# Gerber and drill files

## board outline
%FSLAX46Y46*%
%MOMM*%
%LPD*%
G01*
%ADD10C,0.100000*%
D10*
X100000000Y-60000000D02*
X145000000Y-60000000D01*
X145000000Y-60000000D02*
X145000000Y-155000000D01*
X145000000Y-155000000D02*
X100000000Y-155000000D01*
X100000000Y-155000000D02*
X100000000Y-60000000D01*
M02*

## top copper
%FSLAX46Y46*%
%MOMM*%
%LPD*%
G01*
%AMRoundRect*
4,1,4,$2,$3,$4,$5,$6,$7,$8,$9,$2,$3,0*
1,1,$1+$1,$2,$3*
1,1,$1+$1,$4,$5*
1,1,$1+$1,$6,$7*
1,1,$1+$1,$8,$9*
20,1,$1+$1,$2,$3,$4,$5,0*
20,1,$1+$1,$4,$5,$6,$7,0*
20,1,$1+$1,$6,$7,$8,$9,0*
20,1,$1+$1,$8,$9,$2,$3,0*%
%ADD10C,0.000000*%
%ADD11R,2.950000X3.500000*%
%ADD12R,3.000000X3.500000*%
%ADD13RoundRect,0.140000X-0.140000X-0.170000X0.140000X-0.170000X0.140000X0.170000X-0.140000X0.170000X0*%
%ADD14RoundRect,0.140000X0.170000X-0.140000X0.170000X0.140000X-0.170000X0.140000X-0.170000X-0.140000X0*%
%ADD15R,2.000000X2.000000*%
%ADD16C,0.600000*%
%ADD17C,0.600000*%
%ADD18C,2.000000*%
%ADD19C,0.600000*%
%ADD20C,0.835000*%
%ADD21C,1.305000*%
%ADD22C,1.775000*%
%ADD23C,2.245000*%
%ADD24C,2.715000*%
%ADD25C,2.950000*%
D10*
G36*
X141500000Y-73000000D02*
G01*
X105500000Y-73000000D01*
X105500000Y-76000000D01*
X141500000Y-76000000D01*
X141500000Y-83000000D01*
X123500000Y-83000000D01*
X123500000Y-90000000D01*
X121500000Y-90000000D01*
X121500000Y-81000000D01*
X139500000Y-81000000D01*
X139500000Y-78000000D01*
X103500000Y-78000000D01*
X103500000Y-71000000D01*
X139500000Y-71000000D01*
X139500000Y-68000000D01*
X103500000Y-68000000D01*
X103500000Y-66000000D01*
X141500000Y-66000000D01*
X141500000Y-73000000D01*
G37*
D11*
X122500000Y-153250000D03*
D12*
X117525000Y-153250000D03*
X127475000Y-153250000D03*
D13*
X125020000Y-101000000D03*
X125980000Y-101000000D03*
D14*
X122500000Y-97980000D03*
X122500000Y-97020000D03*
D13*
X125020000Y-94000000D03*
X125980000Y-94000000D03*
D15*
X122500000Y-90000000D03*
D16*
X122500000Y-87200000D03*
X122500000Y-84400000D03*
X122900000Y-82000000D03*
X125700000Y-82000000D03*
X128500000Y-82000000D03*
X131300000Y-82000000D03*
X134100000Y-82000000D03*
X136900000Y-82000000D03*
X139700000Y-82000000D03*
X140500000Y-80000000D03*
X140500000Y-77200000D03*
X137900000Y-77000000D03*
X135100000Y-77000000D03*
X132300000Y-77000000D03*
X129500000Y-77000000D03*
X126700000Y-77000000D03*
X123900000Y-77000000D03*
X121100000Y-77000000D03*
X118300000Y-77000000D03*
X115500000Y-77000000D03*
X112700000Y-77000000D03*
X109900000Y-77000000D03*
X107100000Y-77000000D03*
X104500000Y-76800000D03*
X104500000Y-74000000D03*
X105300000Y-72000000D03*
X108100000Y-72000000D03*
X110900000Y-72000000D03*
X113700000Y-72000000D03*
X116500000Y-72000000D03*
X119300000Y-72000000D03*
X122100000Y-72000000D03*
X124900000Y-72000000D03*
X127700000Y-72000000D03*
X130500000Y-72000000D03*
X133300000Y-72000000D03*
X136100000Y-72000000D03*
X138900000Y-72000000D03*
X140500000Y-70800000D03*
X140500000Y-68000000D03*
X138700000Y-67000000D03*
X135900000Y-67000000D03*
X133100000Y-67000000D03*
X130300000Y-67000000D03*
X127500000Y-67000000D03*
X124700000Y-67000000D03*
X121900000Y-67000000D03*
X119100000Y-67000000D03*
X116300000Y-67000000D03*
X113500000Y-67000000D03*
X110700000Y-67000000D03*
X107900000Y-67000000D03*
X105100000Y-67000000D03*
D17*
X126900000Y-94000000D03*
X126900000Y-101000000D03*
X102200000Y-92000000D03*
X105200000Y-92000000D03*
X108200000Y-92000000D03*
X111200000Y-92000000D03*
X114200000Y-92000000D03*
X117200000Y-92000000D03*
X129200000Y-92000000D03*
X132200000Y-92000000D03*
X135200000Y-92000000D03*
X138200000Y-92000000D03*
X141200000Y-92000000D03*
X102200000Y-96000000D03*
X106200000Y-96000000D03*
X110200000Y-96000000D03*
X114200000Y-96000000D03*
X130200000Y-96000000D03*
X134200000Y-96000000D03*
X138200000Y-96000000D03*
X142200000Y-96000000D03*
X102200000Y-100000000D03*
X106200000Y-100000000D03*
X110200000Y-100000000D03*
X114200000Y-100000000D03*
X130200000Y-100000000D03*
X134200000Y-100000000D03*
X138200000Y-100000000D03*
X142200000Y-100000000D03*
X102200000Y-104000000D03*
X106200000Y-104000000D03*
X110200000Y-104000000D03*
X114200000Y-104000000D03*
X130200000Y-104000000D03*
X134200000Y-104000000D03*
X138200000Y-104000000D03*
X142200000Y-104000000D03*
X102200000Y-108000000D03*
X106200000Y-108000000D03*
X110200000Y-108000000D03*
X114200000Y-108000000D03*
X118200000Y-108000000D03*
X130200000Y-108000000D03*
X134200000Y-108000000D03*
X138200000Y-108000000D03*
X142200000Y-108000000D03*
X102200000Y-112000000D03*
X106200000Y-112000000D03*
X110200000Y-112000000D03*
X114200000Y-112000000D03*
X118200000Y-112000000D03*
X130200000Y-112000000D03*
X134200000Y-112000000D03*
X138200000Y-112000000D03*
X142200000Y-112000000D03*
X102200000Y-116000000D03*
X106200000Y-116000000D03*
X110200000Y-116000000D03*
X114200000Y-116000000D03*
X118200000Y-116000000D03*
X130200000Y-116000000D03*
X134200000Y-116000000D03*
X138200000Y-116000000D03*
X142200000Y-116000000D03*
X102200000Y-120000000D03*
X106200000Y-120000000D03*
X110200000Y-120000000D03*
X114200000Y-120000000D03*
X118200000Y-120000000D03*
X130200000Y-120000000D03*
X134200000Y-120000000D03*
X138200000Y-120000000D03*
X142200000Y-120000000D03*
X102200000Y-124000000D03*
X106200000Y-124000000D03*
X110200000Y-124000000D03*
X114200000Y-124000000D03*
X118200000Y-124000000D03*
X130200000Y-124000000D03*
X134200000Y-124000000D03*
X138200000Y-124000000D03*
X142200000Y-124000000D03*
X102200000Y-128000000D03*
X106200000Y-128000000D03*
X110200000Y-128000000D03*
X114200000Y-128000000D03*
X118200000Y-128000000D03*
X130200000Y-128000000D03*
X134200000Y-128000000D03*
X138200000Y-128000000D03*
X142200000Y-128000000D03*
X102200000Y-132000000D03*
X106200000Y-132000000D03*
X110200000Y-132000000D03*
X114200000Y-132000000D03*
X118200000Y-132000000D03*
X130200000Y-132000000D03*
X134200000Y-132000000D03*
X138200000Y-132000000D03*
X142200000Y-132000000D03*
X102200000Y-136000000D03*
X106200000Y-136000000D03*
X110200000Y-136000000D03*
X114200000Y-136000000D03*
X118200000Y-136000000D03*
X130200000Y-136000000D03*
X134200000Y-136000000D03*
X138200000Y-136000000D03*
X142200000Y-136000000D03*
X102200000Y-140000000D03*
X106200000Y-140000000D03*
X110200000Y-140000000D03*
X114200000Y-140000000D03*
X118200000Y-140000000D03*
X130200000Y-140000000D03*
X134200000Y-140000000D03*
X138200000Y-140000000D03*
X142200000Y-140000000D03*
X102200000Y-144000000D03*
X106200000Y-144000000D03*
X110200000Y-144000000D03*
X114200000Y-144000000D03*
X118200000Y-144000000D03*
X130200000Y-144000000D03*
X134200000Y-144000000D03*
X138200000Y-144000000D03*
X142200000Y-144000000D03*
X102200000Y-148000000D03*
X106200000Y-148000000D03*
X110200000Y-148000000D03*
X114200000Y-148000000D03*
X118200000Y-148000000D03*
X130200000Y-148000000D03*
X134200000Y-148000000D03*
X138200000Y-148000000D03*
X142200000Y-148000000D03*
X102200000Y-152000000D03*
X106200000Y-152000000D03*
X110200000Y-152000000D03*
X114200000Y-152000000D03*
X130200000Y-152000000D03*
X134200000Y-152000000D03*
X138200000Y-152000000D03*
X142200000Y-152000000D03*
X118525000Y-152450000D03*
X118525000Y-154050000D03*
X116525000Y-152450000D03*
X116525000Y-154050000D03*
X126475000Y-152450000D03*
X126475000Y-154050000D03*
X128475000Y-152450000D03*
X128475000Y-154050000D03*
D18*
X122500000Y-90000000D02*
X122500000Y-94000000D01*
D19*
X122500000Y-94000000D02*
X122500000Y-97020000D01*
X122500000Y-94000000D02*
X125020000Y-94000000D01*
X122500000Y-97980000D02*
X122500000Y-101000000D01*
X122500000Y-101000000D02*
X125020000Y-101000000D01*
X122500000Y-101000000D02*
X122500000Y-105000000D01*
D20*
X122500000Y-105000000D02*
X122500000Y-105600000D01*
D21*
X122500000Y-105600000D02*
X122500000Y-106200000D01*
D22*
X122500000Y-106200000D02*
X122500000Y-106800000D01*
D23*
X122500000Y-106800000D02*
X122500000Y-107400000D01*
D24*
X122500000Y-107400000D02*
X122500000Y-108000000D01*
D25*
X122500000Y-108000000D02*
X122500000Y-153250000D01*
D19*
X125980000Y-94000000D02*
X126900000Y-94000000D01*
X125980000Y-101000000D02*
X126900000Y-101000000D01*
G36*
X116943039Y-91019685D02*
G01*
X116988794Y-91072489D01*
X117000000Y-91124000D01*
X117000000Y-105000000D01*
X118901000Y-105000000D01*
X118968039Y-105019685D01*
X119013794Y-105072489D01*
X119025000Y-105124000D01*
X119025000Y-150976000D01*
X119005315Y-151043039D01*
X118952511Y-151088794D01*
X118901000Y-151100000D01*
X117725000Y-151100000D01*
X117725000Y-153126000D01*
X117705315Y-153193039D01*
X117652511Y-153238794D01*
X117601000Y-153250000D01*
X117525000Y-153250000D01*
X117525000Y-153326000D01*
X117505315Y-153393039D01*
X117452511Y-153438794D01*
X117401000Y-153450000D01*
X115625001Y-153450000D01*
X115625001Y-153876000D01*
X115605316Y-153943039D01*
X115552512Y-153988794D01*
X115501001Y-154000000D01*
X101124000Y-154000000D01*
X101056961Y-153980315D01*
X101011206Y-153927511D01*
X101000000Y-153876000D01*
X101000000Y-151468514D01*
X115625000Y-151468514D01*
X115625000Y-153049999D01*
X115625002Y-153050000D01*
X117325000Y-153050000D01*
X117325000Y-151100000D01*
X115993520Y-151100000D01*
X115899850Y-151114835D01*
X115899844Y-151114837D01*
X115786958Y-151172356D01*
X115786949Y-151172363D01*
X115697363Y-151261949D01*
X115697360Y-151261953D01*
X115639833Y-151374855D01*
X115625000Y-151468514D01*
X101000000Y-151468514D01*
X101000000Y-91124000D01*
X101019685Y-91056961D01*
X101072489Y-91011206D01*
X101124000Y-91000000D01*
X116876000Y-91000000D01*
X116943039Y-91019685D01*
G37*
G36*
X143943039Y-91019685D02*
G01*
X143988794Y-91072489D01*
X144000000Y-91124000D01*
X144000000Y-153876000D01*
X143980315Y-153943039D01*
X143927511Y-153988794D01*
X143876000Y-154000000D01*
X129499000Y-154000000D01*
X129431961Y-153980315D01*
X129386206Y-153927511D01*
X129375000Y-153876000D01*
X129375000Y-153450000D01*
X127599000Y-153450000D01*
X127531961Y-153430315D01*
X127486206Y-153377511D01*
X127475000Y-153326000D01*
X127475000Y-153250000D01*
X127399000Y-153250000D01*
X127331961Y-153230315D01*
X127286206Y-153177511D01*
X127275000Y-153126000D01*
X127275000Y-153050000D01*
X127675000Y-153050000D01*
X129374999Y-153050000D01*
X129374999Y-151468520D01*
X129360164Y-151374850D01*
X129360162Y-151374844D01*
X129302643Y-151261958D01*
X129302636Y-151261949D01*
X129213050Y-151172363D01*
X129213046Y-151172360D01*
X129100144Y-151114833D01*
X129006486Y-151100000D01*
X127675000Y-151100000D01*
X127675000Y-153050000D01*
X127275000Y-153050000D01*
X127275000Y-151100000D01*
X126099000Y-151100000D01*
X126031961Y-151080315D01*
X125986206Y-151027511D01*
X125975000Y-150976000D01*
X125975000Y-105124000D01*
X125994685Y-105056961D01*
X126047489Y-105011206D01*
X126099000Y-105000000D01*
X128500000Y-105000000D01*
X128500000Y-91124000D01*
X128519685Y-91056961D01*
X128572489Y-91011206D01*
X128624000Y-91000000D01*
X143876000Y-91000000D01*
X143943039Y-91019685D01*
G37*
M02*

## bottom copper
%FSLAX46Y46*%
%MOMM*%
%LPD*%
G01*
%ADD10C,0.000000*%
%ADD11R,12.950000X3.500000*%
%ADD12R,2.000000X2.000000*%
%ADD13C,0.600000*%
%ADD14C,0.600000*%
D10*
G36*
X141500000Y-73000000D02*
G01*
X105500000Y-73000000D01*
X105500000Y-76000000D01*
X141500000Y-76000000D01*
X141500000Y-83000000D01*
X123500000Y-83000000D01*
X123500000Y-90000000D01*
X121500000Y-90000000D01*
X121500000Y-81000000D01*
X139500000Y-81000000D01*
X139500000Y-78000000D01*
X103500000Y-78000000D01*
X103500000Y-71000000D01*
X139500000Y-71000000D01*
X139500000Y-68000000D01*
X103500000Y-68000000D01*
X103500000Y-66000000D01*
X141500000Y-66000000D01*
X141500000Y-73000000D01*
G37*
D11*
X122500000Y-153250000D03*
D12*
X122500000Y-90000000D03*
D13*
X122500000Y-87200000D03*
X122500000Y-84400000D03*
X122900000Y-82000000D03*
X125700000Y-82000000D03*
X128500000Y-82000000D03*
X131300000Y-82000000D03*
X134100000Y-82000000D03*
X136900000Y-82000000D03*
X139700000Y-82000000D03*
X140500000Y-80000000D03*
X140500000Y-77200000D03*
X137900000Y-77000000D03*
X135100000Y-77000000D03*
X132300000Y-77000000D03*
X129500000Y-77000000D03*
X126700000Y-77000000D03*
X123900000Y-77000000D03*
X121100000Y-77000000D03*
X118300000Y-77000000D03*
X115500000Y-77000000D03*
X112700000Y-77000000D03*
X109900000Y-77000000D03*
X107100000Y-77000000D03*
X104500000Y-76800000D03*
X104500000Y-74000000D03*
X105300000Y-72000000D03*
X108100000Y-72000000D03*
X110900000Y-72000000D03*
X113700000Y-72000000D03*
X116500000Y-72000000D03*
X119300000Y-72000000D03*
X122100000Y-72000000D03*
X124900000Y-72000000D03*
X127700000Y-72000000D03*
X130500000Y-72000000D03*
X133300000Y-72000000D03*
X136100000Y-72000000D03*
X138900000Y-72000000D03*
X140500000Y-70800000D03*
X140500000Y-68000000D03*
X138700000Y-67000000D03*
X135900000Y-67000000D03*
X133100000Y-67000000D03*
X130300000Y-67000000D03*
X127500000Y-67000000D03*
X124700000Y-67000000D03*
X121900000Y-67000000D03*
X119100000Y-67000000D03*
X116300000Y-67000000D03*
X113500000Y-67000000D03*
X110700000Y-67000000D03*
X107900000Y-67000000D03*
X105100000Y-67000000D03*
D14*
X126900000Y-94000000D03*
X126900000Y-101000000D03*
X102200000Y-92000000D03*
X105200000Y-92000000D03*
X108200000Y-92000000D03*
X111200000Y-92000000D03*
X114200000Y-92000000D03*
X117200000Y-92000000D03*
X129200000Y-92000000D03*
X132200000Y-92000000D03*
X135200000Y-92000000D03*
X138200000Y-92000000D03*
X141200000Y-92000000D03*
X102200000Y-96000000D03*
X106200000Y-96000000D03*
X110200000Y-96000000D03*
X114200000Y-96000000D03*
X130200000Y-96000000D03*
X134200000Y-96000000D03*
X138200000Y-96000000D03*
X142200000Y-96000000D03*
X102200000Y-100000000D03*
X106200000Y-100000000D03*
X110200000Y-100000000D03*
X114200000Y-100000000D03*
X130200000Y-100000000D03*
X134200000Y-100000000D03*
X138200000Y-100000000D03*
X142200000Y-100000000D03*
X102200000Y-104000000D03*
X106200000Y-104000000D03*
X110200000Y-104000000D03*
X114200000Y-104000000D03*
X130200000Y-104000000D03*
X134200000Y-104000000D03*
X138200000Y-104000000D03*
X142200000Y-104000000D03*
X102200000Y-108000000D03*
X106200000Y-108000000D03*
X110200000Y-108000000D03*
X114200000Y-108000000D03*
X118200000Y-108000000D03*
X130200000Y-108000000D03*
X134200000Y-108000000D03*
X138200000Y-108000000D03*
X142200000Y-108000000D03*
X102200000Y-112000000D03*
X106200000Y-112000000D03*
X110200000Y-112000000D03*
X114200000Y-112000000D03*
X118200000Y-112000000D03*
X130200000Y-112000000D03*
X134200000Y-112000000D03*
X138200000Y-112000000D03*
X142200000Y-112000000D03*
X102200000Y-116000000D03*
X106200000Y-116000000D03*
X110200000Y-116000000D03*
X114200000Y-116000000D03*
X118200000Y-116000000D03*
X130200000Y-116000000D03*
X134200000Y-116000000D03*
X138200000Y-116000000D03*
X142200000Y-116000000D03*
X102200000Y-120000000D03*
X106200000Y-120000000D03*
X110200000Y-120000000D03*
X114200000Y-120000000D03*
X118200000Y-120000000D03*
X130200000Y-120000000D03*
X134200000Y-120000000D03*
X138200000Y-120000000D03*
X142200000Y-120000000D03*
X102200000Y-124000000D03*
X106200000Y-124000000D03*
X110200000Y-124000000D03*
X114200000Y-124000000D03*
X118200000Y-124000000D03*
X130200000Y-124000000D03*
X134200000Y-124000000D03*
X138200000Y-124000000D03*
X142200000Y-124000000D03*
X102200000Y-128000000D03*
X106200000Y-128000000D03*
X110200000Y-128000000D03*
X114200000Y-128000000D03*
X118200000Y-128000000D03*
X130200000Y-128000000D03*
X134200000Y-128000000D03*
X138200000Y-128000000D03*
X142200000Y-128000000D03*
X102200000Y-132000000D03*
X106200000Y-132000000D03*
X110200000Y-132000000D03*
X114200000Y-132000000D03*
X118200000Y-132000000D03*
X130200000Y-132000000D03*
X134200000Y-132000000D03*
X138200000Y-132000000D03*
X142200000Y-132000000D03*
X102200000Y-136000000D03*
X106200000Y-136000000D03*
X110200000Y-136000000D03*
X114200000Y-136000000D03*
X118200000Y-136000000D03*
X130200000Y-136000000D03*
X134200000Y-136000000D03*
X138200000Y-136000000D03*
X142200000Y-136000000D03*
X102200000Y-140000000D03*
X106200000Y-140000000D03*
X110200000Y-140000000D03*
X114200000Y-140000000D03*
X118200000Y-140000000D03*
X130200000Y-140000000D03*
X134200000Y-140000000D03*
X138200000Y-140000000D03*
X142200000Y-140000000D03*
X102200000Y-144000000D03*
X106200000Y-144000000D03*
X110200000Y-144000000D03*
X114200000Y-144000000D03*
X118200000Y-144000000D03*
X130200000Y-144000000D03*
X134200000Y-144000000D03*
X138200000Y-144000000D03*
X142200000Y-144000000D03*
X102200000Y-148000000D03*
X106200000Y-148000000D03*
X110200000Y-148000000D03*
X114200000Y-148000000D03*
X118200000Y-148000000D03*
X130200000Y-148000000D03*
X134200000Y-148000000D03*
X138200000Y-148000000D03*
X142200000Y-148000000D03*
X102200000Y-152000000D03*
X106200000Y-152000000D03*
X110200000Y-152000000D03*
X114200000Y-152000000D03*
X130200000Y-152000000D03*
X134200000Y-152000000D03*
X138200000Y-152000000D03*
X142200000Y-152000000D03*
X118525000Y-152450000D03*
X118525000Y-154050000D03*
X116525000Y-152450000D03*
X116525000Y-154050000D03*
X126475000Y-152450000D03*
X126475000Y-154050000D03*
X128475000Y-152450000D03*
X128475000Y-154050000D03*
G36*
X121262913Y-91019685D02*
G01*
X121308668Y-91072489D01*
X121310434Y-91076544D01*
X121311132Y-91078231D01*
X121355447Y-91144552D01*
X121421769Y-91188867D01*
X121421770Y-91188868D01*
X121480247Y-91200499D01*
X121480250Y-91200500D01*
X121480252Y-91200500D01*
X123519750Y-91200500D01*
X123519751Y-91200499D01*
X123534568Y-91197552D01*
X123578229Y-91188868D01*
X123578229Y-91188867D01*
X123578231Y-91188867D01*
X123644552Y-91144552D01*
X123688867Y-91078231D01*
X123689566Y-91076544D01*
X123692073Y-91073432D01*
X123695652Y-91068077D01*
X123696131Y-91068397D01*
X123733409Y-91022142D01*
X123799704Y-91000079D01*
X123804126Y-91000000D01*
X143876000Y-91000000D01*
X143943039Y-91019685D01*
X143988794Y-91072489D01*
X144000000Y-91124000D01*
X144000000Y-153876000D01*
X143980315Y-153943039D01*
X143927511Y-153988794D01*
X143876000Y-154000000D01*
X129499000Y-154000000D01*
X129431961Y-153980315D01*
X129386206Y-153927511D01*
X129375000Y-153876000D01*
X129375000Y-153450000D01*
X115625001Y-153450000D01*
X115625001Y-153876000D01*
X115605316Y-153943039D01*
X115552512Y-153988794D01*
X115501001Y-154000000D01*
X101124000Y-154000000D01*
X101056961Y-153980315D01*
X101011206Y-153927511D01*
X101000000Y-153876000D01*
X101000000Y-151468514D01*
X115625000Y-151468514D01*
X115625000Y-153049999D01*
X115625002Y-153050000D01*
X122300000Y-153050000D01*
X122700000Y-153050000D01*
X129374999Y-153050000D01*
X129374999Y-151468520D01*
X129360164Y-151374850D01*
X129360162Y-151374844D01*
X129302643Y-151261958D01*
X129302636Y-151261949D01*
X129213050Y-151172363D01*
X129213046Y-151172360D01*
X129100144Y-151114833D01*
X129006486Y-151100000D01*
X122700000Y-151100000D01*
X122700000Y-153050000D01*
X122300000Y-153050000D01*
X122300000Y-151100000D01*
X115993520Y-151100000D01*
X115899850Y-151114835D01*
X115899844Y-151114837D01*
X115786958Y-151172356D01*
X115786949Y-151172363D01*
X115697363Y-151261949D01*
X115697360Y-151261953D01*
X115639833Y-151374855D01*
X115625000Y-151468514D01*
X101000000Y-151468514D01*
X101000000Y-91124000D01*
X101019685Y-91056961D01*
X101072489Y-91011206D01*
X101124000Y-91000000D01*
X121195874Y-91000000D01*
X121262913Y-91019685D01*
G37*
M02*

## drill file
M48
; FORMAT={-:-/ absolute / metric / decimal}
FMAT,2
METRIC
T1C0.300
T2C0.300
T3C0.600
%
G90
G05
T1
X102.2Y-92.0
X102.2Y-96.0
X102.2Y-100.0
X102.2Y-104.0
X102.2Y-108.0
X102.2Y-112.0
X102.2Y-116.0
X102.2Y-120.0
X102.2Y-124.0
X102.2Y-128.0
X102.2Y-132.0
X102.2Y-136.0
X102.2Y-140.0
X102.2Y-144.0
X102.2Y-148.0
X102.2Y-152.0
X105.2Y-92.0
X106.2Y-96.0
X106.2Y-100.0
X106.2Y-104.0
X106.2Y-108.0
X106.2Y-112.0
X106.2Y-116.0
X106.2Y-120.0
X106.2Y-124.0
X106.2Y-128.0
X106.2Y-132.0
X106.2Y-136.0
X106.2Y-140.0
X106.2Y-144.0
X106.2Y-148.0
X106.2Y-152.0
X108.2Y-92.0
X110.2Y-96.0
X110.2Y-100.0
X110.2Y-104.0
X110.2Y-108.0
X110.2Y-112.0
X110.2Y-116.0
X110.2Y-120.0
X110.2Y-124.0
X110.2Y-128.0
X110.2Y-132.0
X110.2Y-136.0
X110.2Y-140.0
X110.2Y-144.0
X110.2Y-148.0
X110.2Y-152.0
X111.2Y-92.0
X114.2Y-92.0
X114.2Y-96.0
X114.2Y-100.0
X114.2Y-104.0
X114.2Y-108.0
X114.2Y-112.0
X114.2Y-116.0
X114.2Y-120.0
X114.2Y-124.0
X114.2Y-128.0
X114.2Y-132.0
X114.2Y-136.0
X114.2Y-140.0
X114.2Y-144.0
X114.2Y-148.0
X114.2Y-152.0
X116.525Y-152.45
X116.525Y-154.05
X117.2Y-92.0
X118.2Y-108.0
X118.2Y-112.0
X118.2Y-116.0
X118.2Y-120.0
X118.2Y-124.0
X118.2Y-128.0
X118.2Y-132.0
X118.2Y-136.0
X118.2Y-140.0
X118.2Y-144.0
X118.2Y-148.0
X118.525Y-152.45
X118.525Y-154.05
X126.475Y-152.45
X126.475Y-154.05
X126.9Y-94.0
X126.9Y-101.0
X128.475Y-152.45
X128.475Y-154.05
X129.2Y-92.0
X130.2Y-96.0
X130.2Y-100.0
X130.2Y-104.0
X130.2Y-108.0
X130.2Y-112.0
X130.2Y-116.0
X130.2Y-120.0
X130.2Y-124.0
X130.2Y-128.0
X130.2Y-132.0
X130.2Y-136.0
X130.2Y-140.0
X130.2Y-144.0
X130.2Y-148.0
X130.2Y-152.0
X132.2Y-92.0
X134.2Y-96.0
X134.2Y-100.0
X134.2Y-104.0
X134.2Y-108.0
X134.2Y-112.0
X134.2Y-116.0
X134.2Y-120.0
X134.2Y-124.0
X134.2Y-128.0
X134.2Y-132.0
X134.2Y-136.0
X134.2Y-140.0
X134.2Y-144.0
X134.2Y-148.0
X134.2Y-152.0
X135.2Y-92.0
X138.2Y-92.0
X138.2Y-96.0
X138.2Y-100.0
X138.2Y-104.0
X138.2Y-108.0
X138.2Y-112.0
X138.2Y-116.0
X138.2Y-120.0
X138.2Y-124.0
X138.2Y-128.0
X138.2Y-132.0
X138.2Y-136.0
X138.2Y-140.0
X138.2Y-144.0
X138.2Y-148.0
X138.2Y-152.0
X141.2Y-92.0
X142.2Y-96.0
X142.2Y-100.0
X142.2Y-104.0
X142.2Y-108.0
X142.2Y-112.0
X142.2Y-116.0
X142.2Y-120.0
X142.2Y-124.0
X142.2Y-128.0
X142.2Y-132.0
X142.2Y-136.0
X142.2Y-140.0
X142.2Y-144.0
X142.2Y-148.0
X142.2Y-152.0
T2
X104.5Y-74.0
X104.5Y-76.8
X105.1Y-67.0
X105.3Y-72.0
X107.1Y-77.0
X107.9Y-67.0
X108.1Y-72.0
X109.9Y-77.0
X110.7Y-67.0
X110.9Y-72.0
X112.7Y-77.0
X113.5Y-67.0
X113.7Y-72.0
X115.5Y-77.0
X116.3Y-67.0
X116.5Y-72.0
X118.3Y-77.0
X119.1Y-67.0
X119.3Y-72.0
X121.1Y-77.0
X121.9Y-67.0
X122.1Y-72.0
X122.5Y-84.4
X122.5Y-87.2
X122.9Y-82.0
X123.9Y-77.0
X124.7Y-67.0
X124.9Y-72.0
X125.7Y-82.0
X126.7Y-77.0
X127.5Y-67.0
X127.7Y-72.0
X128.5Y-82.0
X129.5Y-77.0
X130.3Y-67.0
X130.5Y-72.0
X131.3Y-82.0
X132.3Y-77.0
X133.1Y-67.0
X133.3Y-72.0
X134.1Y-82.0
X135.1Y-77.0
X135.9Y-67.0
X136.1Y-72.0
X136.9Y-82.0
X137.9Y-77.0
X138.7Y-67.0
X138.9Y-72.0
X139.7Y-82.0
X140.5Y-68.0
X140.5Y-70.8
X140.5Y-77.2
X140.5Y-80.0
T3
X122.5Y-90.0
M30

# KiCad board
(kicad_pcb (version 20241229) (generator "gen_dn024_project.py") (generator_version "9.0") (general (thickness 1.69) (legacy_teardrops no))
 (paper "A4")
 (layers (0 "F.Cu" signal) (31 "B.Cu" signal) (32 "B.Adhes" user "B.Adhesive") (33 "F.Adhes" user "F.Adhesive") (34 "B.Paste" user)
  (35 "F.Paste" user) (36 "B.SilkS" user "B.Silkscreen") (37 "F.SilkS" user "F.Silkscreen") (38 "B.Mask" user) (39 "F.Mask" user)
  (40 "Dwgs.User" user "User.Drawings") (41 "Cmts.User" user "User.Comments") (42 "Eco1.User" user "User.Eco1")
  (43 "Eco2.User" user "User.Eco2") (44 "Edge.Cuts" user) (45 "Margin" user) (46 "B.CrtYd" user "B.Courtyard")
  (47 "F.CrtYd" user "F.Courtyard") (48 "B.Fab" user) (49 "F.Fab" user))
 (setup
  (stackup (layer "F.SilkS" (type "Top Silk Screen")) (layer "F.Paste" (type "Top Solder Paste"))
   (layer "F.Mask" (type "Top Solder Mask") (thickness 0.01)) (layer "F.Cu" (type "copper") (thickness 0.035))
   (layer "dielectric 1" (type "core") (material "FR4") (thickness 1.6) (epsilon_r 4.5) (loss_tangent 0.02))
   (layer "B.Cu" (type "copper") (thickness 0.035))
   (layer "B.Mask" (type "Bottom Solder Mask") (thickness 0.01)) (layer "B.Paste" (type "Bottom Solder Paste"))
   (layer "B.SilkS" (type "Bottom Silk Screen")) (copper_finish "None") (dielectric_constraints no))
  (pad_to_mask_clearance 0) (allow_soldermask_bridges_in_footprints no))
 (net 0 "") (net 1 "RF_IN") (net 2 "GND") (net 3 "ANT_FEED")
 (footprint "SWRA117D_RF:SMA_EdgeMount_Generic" (layer "F.Cu") (at 122.5 155 90)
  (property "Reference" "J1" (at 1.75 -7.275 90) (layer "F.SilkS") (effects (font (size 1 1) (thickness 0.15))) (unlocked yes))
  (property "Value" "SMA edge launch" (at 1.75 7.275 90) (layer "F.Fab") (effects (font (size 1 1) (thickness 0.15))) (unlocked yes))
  (pad "1" smd rect (at 1.75 0 90) (size 3.5 2.95) (layers "F.Cu" "F.Paste" "F.Mask") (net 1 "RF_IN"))
  (pad "2" smd rect (at 1.75 -4.975 90) (size 3.5 3) (layers "F.Cu" "F.Paste" "F.Mask") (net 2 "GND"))
  (pad "2" smd rect (at 1.75 4.975 90) (size 3.5 3) (layers "F.Cu" "F.Paste" "F.Mask") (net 2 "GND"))
  (pad "2" smd rect (at 1.75 0 90) (size 3.5 12.95) (layers "B.Cu" "B.Paste" "B.Mask") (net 2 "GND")))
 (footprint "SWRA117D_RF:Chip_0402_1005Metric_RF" (layer "F.Cu") (at 125.5 101)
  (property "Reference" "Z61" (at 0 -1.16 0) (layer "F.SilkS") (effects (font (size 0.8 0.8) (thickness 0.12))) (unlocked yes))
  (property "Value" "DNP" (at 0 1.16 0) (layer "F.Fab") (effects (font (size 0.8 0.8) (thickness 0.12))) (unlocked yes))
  (pad "1" smd roundrect (at -0.48 0) (size 0.56 0.62) (layers "F.Cu" "F.Paste" "F.Mask") (roundrect_rratio 0.25) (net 1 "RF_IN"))
  (pad "2" smd roundrect (at 0.48 0) (size 0.56 0.62) (layers "F.Cu" "F.Paste" "F.Mask") (roundrect_rratio 0.25) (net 2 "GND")))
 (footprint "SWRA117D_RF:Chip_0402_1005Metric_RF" (layer "F.Cu") (at 122.5 97.5 90)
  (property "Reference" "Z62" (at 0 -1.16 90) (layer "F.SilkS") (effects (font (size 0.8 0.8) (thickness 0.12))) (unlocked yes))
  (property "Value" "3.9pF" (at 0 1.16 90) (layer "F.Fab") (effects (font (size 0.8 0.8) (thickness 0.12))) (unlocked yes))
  (pad "1" smd roundrect (at -0.48 0 90) (size 0.56 0.62) (layers "F.Cu" "F.Paste" "F.Mask") (roundrect_rratio 0.25) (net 1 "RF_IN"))
  (pad "2" smd roundrect (at 0.48 0 90) (size 0.56 0.62) (layers "F.Cu" "F.Paste" "F.Mask") (roundrect_rratio 0.25) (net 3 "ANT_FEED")))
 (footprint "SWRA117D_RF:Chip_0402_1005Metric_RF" (layer "F.Cu") (at 125.5 94)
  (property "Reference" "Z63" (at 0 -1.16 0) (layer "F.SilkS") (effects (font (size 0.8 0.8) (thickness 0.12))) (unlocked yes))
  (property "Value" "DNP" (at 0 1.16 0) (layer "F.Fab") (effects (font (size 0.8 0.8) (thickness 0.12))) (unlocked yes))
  (pad "1" smd roundrect (at -0.48 0) (size 0.56 0.62) (layers "F.Cu" "F.Paste" "F.Mask") (roundrect_rratio 0.25) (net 3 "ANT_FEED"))
  (pad "2" smd roundrect (at 0.48 0) (size 0.56 0.62) (layers "F.Cu" "F.Paste" "F.Mask") (roundrect_rratio 0.25) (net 2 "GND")))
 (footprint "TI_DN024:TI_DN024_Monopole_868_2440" (layer "F.Cu") (at 122.5 90)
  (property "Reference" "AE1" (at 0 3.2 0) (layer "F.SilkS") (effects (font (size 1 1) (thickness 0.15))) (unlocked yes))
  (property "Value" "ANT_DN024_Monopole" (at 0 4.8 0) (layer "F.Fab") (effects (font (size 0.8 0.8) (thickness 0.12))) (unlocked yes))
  (fp_poly
   (pts (xy 1 0) (xy 1 -7) (xy 19 -7) (xy 19 -14) (xy -17 -14) (xy -17 -17) (xy 19 -17) (xy 19 -24) (xy -19 -24) (xy -19 -22) (xy 17 -22)
    (xy 17 -19) (xy -19 -19) (xy -19 -12) (xy 17 -12) (xy 17 -9) (xy -1 -9) (xy -1 0))
   (stroke (width 0) (type solid)) (fill yes) (layer "F.Cu"))
  (fp_poly
   (pts (xy 1 0) (xy 1 -7) (xy 19 -7) (xy 19 -14) (xy -17 -14) (xy -17 -17) (xy 19 -17) (xy 19 -24) (xy -19 -24) (xy -19 -22) (xy 17 -22)
    (xy 17 -19) (xy -19 -19) (xy -19 -12) (xy 17 -12) (xy 17 -9) (xy -1 -9) (xy -1 0))
   (stroke (width 0) (type solid)) (fill yes) (layer "B.Cu"))
  (pad "1" thru_hole rect (at 0 0) (size 2 2) (drill 0.6) (layers "*.Cu" "*.Mask") (remove_unused_layers no) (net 3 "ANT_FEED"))
  (pad "1" thru_hole circle (at 0 -2.8) (size 0.6 0.6) (drill 0.3) (layers "*.Cu") (remove_unused_layers no) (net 3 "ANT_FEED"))
  (pad "1" thru_hole circle (at 0 -5.6) (size 0.6 0.6) (drill 0.3) (layers "*.Cu") (remove_unused_layers no) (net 3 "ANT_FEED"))
  (pad "1" thru_hole circle (at 0.4 -8) (size 0.6 0.6) (drill 0.3) (layers "*.Cu") (remove_unused_layers no) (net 3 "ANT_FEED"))
  (pad "1" thru_hole circle (at 3.2 -8) (size 0.6 0.6) (drill 0.3) (layers "*.Cu") (remove_unused_layers no) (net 3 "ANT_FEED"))
  (pad "1" thru_hole circle (at 6 -8) (size 0.6 0.6) (drill 0.3) (layers "*.Cu") (remove_unused_layers no) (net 3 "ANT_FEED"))
  (pad "1" thru_hole circle (at 8.8 -8) (size 0.6 0.6) (drill 0.3) (layers "*.Cu") (remove_unused_layers no) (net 3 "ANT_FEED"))
  (pad "1" thru_hole circle (at 11.6 -8) (size 0.6 0.6) (drill 0.3) (layers "*.Cu") (remove_unused_layers no) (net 3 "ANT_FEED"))
  (pad "1" thru_hole circle (at 14.4 -8) (size 0.6 0.6) (drill 0.3) (layers "*.Cu") (remove_unused_layers no) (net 3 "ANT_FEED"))
  (pad "1" thru_hole circle (at 17.2 -8) (size 0.6 0.6) (drill 0.3) (layers "*.Cu") (remove_unused_layers no) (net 3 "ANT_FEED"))
  (pad "1" thru_hole circle (at 18 -10) (size 0.6 0.6) (drill 0.3) (layers "*.Cu") (remove_unused_layers no) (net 3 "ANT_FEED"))
  (pad "1" thru_hole circle (at 18 -12.8) (size 0.6 0.6) (drill 0.3) (layers "*.Cu") (remove_unused_layers no) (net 3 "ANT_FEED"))
  (pad "1" thru_hole circle (at 15.4 -13) (size 0.6 0.6) (drill 0.3) (layers "*.Cu") (remove_unused_layers no) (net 3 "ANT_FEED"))
  (pad "1" thru_hole circle (at 12.6 -13) (size 0.6 0.6) (drill 0.3) (layers "*.Cu") (remove_unused_layers no) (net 3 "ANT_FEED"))
  (pad "1" thru_hole circle (at 9.8 -13) (size 0.6 0.6) (drill 0.3) (layers "*.Cu") (remove_unused_layers no) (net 3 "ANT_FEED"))
  (pad "1" thru_hole circle (at 7 -13) (size 0.6 0.6) (drill 0.3) (layers "*.Cu") (remove_unused_layers no) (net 3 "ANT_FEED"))
  (pad "1" thru_hole circle (at 4.2 -13) (size 0.6 0.6) (drill 0.3) (layers "*.Cu") (remove_unused_layers no) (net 3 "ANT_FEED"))
  (pad "1" thru_hole circle (at 1.4 -13) (size 0.6 0.6) (drill 0.3) (layers "*.Cu") (remove_unused_layers no) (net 3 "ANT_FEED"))
  (pad "1" thru_hole circle (at -1.4 -13) (size 0.6 0.6) (drill 0.3) (layers "*.Cu") (remove_unused_layers no) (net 3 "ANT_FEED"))
  (pad "1" thru_hole circle (at -4.2 -13) (size 0.6 0.6) (drill 0.3) (layers "*.Cu") (remove_unused_layers no) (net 3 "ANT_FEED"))
  (pad "1" thru_hole circle (at -7 -13) (size 0.6 0.6) (drill 0.3) (layers "*.Cu") (remove_unused_layers no) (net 3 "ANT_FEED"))
  (pad "1" thru_hole circle (at -9.8 -13) (size 0.6 0.6) (drill 0.3) (layers "*.Cu") (remove_unused_layers no) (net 3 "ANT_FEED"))
  (pad "1" thru_hole circle (at -12.6 -13) (size 0.6 0.6) (drill 0.3) (layers "*.Cu") (remove_unused_layers no) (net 3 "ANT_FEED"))
  (pad "1" thru_hole circle (at -15.4 -13) (size 0.6 0.6) (drill 0.3) (layers "*.Cu") (remove_unused_layers no) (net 3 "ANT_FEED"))
  (pad "1" thru_hole circle (at -18 -13.2) (size 0.6 0.6) (drill 0.3) (layers "*.Cu") (remove_unused_layers no) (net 3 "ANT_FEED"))
  (pad "1" thru_hole circle (at -18 -16) (size 0.6 0.6) (drill 0.3) (layers "*.Cu") (remove_unused_layers no) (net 3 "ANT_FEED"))
  (pad "1" thru_hole circle (at -17.2 -18) (size 0.6 0.6) (drill 0.3) (layers "*.Cu") (remove_unused_layers no) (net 3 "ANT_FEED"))
  (pad "1" thru_hole circle (at -14.4 -18) (size 0.6 0.6) (drill 0.3) (layers "*.Cu") (remove_unused_layers no) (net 3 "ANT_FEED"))
  (pad "1" thru_hole circle (at -11.6 -18) (size 0.6 0.6) (drill 0.3) (layers "*.Cu") (remove_unused_layers no) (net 3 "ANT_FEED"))
  (pad "1" thru_hole circle (at -8.8 -18) (size 0.6 0.6) (drill 0.3) (layers "*.Cu") (remove_unused_layers no) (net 3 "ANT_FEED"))
  (pad "1" thru_hole circle (at -6 -18) (size 0.6 0.6) (drill 0.3) (layers "*.Cu") (remove_unused_layers no) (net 3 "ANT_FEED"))
  (pad "1" thru_hole circle (at -3.2 -18) (size 0.6 0.6) (drill 0.3) (layers "*.Cu") (remove_unused_layers no) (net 3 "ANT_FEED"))
  (pad "1" thru_hole circle (at -0.4 -18) (size 0.6 0.6) (drill 0.3) (layers "*.Cu") (remove_unused_layers no) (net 3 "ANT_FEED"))
  (pad "1" thru_hole circle (at 2.4 -18) (size 0.6 0.6) (drill 0.3) (layers "*.Cu") (remove_unused_layers no) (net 3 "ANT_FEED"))
  (pad "1" thru_hole circle (at 5.2 -18) (size 0.6 0.6) (drill 0.3) (layers "*.Cu") (remove_unused_layers no) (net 3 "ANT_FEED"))
  (pad "1" thru_hole circle (at 8 -18) (size 0.6 0.6) (drill 0.3) (layers "*.Cu") (remove_unused_layers no) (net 3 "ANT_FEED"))
  (pad "1" thru_hole circle (at 10.8 -18) (size 0.6 0.6) (drill 0.3) (layers "*.Cu") (remove_unused_layers no) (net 3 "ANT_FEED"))
  (pad "1" thru_hole circle (at 13.6 -18) (size 0.6 0.6) (drill 0.3) (layers "*.Cu") (remove_unused_layers no) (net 3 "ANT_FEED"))
  (pad "1" thru_hole circle (at 16.4 -18) (size 0.6 0.6) (drill 0.3) (layers "*.Cu") (remove_unused_layers no) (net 3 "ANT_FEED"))
  (pad "1" thru_hole circle (at 18 -19.2) (size 0.6 0.6) (drill 0.3) (layers "*.Cu") (remove_unused_layers no) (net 3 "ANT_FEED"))
  (pad "1" thru_hole circle (at 18 -22) (size 0.6 0.6) (drill 0.3) (layers "*.Cu") (remove_unused_layers no) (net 3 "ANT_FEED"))
  (pad "1" thru_hole circle (at 16.2 -23) (size 0.6 0.6) (drill 0.3) (layers "*.Cu") (remove_unused_layers no) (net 3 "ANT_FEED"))
  (pad "1" thru_hole circle (at 13.4 -23) (size 0.6 0.6) (drill 0.3) (layers "*.Cu") (remove_unused_layers no) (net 3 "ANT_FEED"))
  (pad "1" thru_hole circle (at 10.6 -23) (size 0.6 0.6) (drill 0.3) (layers "*.Cu") (remove_unused_layers no) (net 3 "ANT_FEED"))
  (pad "1" thru_hole circle (at 7.8 -23) (size 0.6 0.6) (drill 0.3) (layers "*.Cu") (remove_unused_layers no) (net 3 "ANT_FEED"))
  (pad "1" thru_hole circle (at 5 -23) (size 0.6 0.6) (drill 0.3) (layers "*.Cu") (remove_unused_layers no) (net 3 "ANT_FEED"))
  (pad "1" thru_hole circle (at 2.2 -23) (size 0.6 0.6) (drill 0.3) (layers "*.Cu") (remove_unused_layers no) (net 3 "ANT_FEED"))
  (pad "1" thru_hole circle (at -0.6 -23) (size 0.6 0.6) (drill 0.3) (layers "*.Cu") (remove_unused_layers no) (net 3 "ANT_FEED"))
  (pad "1" thru_hole circle (at -3.4 -23) (size 0.6 0.6) (drill 0.3) (layers "*.Cu") (remove_unused_layers no) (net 3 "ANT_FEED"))
  (pad "1" thru_hole circle (at -6.2 -23) (size 0.6 0.6) (drill 0.3) (layers "*.Cu") (remove_unused_layers no) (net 3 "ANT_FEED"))
  (pad "1" thru_hole circle (at -9 -23) (size 0.6 0.6) (drill 0.3) (layers "*.Cu") (remove_unused_layers no) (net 3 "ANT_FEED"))
  (pad "1" thru_hole circle (at -11.8 -23) (size 0.6 0.6) (drill 0.3) (layers "*.Cu") (remove_unused_layers no) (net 3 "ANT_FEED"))
  (pad "1" thru_hole circle (at -14.6 -23) (size 0.6 0.6) (drill 0.3) (layers "*.Cu") (remove_unused_layers no) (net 3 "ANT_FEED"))
  (pad "1" thru_hole circle (at -17.4 -23) (size 0.6 0.6) (drill 0.3) (layers "*.Cu") (remove_unused_layers no) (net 3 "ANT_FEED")))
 (gr_line (start 100 60) (end 145 60) (stroke (width 0.1) (type solid)) (layer "Edge.Cuts"))
 (gr_line (start 145 60) (end 145 155) (stroke (width 0.1) (type solid)) (layer "Edge.Cuts"))
 (gr_line (start 145 155) (end 100 155) (stroke (width 0.1) (type solid)) (layer "Edge.Cuts"))
 (gr_line (start 100 155) (end 100 60) (stroke (width 0.1) (type solid)) (layer "Edge.Cuts"))
 (segment (start 122.5 90) (end 122.5 94) (width 2) (layer "F.Cu") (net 3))
 (segment (start 122.5 94) (end 122.5 97.02) (width 0.6) (layer "F.Cu") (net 3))
 (segment (start 122.5 94) (end 125.02 94) (width 0.6) (layer "F.Cu") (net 3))
 (segment (start 122.5 97.98) (end 122.5 101) (width 0.6) (layer "F.Cu") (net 1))
 (segment (start 122.5 101) (end 125.02 101) (width 0.6) (layer "F.Cu") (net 1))
 (segment (start 122.5 101) (end 122.5 105) (width 0.6) (layer "F.Cu") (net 1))
 (segment (start 122.5 105) (end 122.5 105.6) (width 0.835) (layer "F.Cu") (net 1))
 (segment (start 122.5 105.6) (end 122.5 106.2) (width 1.305) (layer "F.Cu") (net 1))
 (segment (start 122.5 106.2) (end 122.5 106.8) (width 1.775) (layer "F.Cu") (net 1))
 (segment (start 122.5 106.8) (end 122.5 107.4) (width 2.245) (layer "F.Cu") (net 1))
 (segment (start 122.5 107.4) (end 122.5 108) (width 2.715) (layer "F.Cu") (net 1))
 (segment (start 122.5 108) (end 122.5 153.25) (width 2.95) (layer "F.Cu") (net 1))
 (segment (start 125.98 94) (end 126.9 94) (width 0.6) (layer "F.Cu") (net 2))
 (segment (start 125.98 101) (end 126.9 101) (width 0.6) (layer "F.Cu") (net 2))
 (via (at 126.9 94) (size 0.6) (drill 0.3) (layers "F.Cu" "B.Cu") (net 2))
 (via (at 126.9 101) (size 0.6) (drill 0.3) (layers "F.Cu" "B.Cu") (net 2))
 (via (at 102.2 92) (size 0.6) (drill 0.3) (layers "F.Cu" "B.Cu") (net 2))
 (via (at 105.2 92) (size 0.6) (drill 0.3) (layers "F.Cu" "B.Cu") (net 2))
 (via (at 108.2 92) (size 0.6) (drill 0.3) (layers "F.Cu" "B.Cu") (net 2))
 (via (at 111.2 92) (size 0.6) (drill 0.3) (layers "F.Cu" "B.Cu") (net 2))
 (via (at 114.2 92) (size 0.6) (drill 0.3) (layers "F.Cu" "B.Cu") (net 2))
 (via (at 117.2 92) (size 0.6) (drill 0.3) (layers "F.Cu" "B.Cu") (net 2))
 (via (at 129.2 92) (size 0.6) (drill 0.3) (layers "F.Cu" "B.Cu") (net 2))
 (via (at 132.2 92) (size 0.6) (drill 0.3) (layers "F.Cu" "B.Cu") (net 2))
 (via (at 135.2 92) (size 0.6) (drill 0.3) (layers "F.Cu" "B.Cu") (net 2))
 (via (at 138.2 92) (size 0.6) (drill 0.3) (layers "F.Cu" "B.Cu") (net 2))
 (via (at 141.2 92) (size 0.6) (drill 0.3) (layers "F.Cu" "B.Cu") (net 2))
 (via (at 102.2 96) (size 0.6) (drill 0.3) (layers "F.Cu" "B.Cu") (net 2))
 (via (at 106.2 96) (size 0.6) (drill 0.3) (layers "F.Cu" "B.Cu") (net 2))
 (via (at 110.2 96) (size 0.6) (drill 0.3) (layers "F.Cu" "B.Cu") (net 2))
 (via (at 114.2 96) (size 0.6) (drill 0.3) (layers "F.Cu" "B.Cu") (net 2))
 (via (at 130.2 96) (size 0.6) (drill 0.3) (layers "F.Cu" "B.Cu") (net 2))
 (via (at 134.2 96) (size 0.6) (drill 0.3) (layers "F.Cu" "B.Cu") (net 2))
 (via (at 138.2 96) (size 0.6) (drill 0.3) (layers "F.Cu" "B.Cu") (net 2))
 (via (at 142.2 96) (size 0.6) (drill 0.3) (layers "F.Cu" "B.Cu") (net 2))
 (via (at 102.2 100) (size 0.6) (drill 0.3) (layers "F.Cu" "B.Cu") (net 2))
 (via (at 106.2 100) (size 0.6) (drill 0.3) (layers "F.Cu" "B.Cu") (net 2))
 (via (at 110.2 100) (size 0.6) (drill 0.3) (layers "F.Cu" "B.Cu") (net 2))
 (via (at 114.2 100) (size 0.6) (drill 0.3) (layers "F.Cu" "B.Cu") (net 2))
 (via (at 130.2 100) (size 0.6) (drill 0.3) (layers "F.Cu" "B.Cu") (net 2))
 (via (at 134.2 100) (size 0.6) (drill 0.3) (layers "F.Cu" "B.Cu") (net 2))
 (via (at 138.2 100) (size 0.6) (drill 0.3) (layers "F.Cu" "B.Cu") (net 2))
 (via (at 142.2 100) (size 0.6) (drill 0.3) (layers "F.Cu" "B.Cu") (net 2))
 (via (at 102.2 104) (size 0.6) (drill 0.3) (layers "F.Cu" "B.Cu") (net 2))
 (via (at 106.2 104) (size 0.6) (drill 0.3) (layers "F.Cu" "B.Cu") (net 2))
 (via (at 110.2 104) (size 0.6) (drill 0.3) (layers "F.Cu" "B.Cu") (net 2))
 (via (at 114.2 104) (size 0.6) (drill 0.3) (layers "F.Cu" "B.Cu") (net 2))
 (via (at 130.2 104) (size 0.6) (drill 0.3) (layers "F.Cu" "B.Cu") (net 2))
 (via (at 134.2 104) (size 0.6) (drill 0.3) (layers "F.Cu" "B.Cu") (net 2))
 (via (at 138.2 104) (size 0.6) (drill 0.3) (layers "F.Cu" "B.Cu") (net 2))
 (via (at 142.2 104) (size 0.6) (drill 0.3) (layers "F.Cu" "B.Cu") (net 2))
 (via (at 102.2 108) (size 0.6) (drill 0.3) (layers "F.Cu" "B.Cu") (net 2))
 (via (at 106.2 108) (size 0.6) (drill 0.3) (layers "F.Cu" "B.Cu") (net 2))
 (via (at 110.2 108) (size 0.6) (drill 0.3) (layers "F.Cu" "B.Cu") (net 2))
 (via (at 114.2 108) (size 0.6) (drill 0.3) (layers "F.Cu" "B.Cu") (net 2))
 (via (at 118.2 108) (size 0.6) (drill 0.3) (layers "F.Cu" "B.Cu") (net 2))
 (via (at 130.2 108) (size 0.6) (drill 0.3) (layers "F.Cu" "B.Cu") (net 2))
 (via (at 134.2 108) (size 0.6) (drill 0.3) (layers "F.Cu" "B.Cu") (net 2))
 (via (at 138.2 108) (size 0.6) (drill 0.3) (layers "F.Cu" "B.Cu") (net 2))
 (via (at 142.2 108) (size 0.6) (drill 0.3) (layers "F.Cu" "B.Cu") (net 2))
 (via (at 102.2 112) (size 0.6) (drill 0.3) (layers "F.Cu" "B.Cu") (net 2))
 (via (at 106.2 112) (size 0.6) (drill 0.3) (layers "F.Cu" "B.Cu") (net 2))
 (via (at 110.2 112) (size 0.6) (drill 0.3) (layers "F.Cu" "B.Cu") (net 2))
 (via (at 114.2 112) (size 0.6) (drill 0.3) (layers "F.Cu" "B.Cu") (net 2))
 (via (at 118.2 112) (size 0.6) (drill 0.3) (layers "F.Cu" "B.Cu") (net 2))
 (via (at 130.2 112) (size 0.6) (drill 0.3) (layers "F.Cu" "B.Cu") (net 2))
 (via (at 134.2 112) (size 0.6) (drill 0.3) (layers "F.Cu" "B.Cu") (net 2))
 (via (at 138.2 112) (size 0.6) (drill 0.3) (layers "F.Cu" "B.Cu") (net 2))
 (via (at 142.2 112) (size 0.6) (drill 0.3) (layers "F.Cu" "B.Cu") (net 2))
 (via (at 102.2 116) (size 0.6) (drill 0.3) (layers "F.Cu" "B.Cu") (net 2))
 (via (at 106.2 116) (size 0.6) (drill 0.3) (layers "F.Cu" "B.Cu") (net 2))
 (via (at 110.2 116) (size 0.6) (drill 0.3) (layers "F.Cu" "B.Cu") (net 2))
 (via (at 114.2 116) (size 0.6) (drill 0.3) (layers "F.Cu" "B.Cu") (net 2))
 (via (at 118.2 116) (size 0.6) (drill 0.3) (layers "F.Cu" "B.Cu") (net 2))
 (via (at 130.2 116) (size 0.6) (drill 0.3) (layers "F.Cu" "B.Cu") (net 2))
 (via (at 134.2 116) (size 0.6) (drill 0.3) (layers "F.Cu" "B.Cu") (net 2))
 (via (at 138.2 116) (size 0.6) (drill 0.3) (layers "F.Cu" "B.Cu") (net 2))
 (via (at 142.2 116) (size 0.6) (drill 0.3) (layers "F.Cu" "B.Cu") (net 2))
 (via (at 102.2 120) (size 0.6) (drill 0.3) (layers "F.Cu" "B.Cu") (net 2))
 (via (at 106.2 120) (size 0.6) (drill 0.3) (layers "F.Cu" "B.Cu") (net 2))
 (via (at 110.2 120) (size 0.6) (drill 0.3) (layers "F.Cu" "B.Cu") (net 2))
 (via (at 114.2 120) (size 0.6) (drill 0.3) (layers "F.Cu" "B.Cu") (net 2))
 (via (at 118.2 120) (size 0.6) (drill 0.3) (layers "F.Cu" "B.Cu") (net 2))
 (via (at 130.2 120) (size 0.6) (drill 0.3) (layers "F.Cu" "B.Cu") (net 2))
 (via (at 134.2 120) (size 0.6) (drill 0.3) (layers "F.Cu" "B.Cu") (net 2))
 (via (at 138.2 120) (size 0.6) (drill 0.3) (layers "F.Cu" "B.Cu") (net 2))
 (via (at 142.2 120) (size 0.6) (drill 0.3) (layers "F.Cu" "B.Cu") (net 2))
 (via (at 102.2 124) (size 0.6) (drill 0.3) (layers "F.Cu" "B.Cu") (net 2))
 (via (at 106.2 124) (size 0.6) (drill 0.3) (layers "F.Cu" "B.Cu") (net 2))
 (via (at 110.2 124) (size 0.6) (drill 0.3) (layers "F.Cu" "B.Cu") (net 2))
 (via (at 114.2 124) (size 0.6) (drill 0.3) (layers "F.Cu" "B.Cu") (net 2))
 (via (at 118.2 124) (size 0.6) (drill 0.3) (layers "F.Cu" "B.Cu") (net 2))
 (via (at 130.2 124) (size 0.6) (drill 0.3) (layers "F.Cu" "B.Cu") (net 2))
 (via (at 134.2 124) (size 0.6) (drill 0.3) (layers "F.Cu" "B.Cu") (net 2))
 (via (at 138.2 124) (size 0.6) (drill 0.3) (layers "F.Cu" "B.Cu") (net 2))
 (via (at 142.2 124) (size 0.6) (drill 0.3) (layers "F.Cu" "B.Cu") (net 2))
 (via (at 102.2 128) (size 0.6) (drill 0.3) (layers "F.Cu" "B.Cu") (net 2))
 (via (at 106.2 128) (size 0.6) (drill 0.3) (layers "F.Cu" "B.Cu") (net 2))
 (via (at 110.2 128) (size 0.6) (drill 0.3) (layers "F.Cu" "B.Cu") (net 2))
 (via (at 114.2 128) (size 0.6) (drill 0.3) (layers "F.Cu" "B.Cu") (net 2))
 (via (at 118.2 128) (size 0.6) (drill 0.3) (layers "F.Cu" "B.Cu") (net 2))
 (via (at 130.2 128) (size 0.6) (drill 0.3) (layers "F.Cu" "B.Cu") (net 2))
 (via (at 134.2 128) (size 0.6) (drill 0.3) (layers "F.Cu" "B.Cu") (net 2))
 (via (at 138.2 128) (size 0.6) (drill 0.3) (layers "F.Cu" "B.Cu") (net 2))
 (via (at 142.2 128) (size 0.6) (drill 0.3) (layers "F.Cu" "B.Cu") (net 2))
 (via (at 102.2 132) (size 0.6) (drill 0.3) (layers "F.Cu" "B.Cu") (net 2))
 (via (at 106.2 132) (size 0.6) (drill 0.3) (layers "F.Cu" "B.Cu") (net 2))
 (via (at 110.2 132) (size 0.6) (drill 0.3) (layers "F.Cu" "B.Cu") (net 2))
 (via (at 114.2 132) (size 0.6) (drill 0.3) (layers "F.Cu" "B.Cu") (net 2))
 (via (at 118.2 132) (size 0.6) (drill 0.3) (layers "F.Cu" "B.Cu") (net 2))
 (via (at 130.2 132) (size 0.6) (drill 0.3) (layers "F.Cu" "B.Cu") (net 2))
 (via (at 134.2 132) (size 0.6) (drill 0.3) (layers "F.Cu" "B.Cu") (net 2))
 (via (at 138.2 132) (size 0.6) (drill 0.3) (layers "F.Cu" "B.Cu") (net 2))
 (via (at 142.2 132) (size 0.6) (drill 0.3) (layers "F.Cu" "B.Cu") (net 2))
 (via (at 102.2 136) (size 0.6) (drill 0.3) (layers "F.Cu" "B.Cu") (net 2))
 (via (at 106.2 136) (size 0.6) (drill 0.3) (layers "F.Cu" "B.Cu") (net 2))
 (via (at 110.2 136) (size 0.6) (drill 0.3) (layers "F.Cu" "B.Cu") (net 2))
 (via (at 114.2 136) (size 0.6) (drill 0.3) (layers "F.Cu" "B.Cu") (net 2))
 (via (at 118.2 136) (size 0.6) (drill 0.3) (layers "F.Cu" "B.Cu") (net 2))
 (via (at 130.2 136) (size 0.6) (drill 0.3) (layers "F.Cu" "B.Cu") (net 2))
 (via (at 134.2 136) (size 0.6) (drill 0.3) (layers "F.Cu" "B.Cu") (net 2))
 (via (at 138.2 136) (size 0.6) (drill 0.3) (layers "F.Cu" "B.Cu") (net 2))
 (via (at 142.2 136) (size 0.6) (drill 0.3) (layers "F.Cu" "B.Cu") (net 2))
 (via (at 102.2 140) (size 0.6) (drill 0.3) (layers "F.Cu" "B.Cu") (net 2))
 (via (at 106.2 140) (size 0.6) (drill 0.3) (layers "F.Cu" "B.Cu") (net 2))
 (via (at 110.2 140) (size 0.6) (drill 0.3) (layers "F.Cu" "B.Cu") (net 2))
 (via (at 114.2 140) (size 0.6) (drill 0.3) (layers "F.Cu" "B.Cu") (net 2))
 (via (at 118.2 140) (size 0.6) (drill 0.3) (layers "F.Cu" "B.Cu") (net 2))
 (via (at 130.2 140) (size 0.6) (drill 0.3) (layers "F.Cu" "B.Cu") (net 2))
 (via (at 134.2 140) (size 0.6) (drill 0.3) (layers "F.Cu" "B.Cu") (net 2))
 (via (at 138.2 140) (size 0.6) (drill 0.3) (layers "F.Cu" "B.Cu") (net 2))
 (via (at 142.2 140) (size 0.6) (drill 0.3) (layers "F.Cu" "B.Cu") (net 2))
 (via (at 102.2 144) (size 0.6) (drill 0.3) (layers "F.Cu" "B.Cu") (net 2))
 (via (at 106.2 144) (size 0.6) (drill 0.3) (layers "F.Cu" "B.Cu") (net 2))
 (via (at 110.2 144) (size 0.6) (drill 0.3) (layers "F.Cu" "B.Cu") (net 2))
 (via (at 114.2 144) (size 0.6) (drill 0.3) (layers "F.Cu" "B.Cu") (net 2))
 (via (at 118.2 144) (size 0.6) (drill 0.3) (layers "F.Cu" "B.Cu") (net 2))
 (via (at 130.2 144) (size 0.6) (drill 0.3) (layers "F.Cu" "B.Cu") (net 2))
 (via (at 134.2 144) (size 0.6) (drill 0.3) (layers "F.Cu" "B.Cu") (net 2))
 (via (at 138.2 144) (size 0.6) (drill 0.3) (layers "F.Cu" "B.Cu") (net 2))
 (via (at 142.2 144) (size 0.6) (drill 0.3) (layers "F.Cu" "B.Cu") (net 2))
 (via (at 102.2 148) (size 0.6) (drill 0.3) (layers "F.Cu" "B.Cu") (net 2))
 (via (at 106.2 148) (size 0.6) (drill 0.3) (layers "F.Cu" "B.Cu") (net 2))
 (via (at 110.2 148) (size 0.6) (drill 0.3) (layers "F.Cu" "B.Cu") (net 2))
 (via (at 114.2 148) (size 0.6) (drill 0.3) (layers "F.Cu" "B.Cu") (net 2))
 (via (at 118.2 148) (size 0.6) (drill 0.3) (layers "F.Cu" "B.Cu") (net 2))
 (via (at 130.2 148) (size 0.6) (drill 0.3) (layers "F.Cu" "B.Cu") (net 2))
 (via (at 134.2 148) (size 0.6) (drill 0.3) (layers "F.Cu" "B.Cu") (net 2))
 (via (at 138.2 148) (size 0.6) (drill 0.3) (layers "F.Cu" "B.Cu") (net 2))
 (via (at 142.2 148) (size 0.6) (drill 0.3) (layers "F.Cu" "B.Cu") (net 2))
 (via (at 102.2 152) (size 0.6) (drill 0.3) (layers "F.Cu" "B.Cu") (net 2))
 (via (at 106.2 152) (size 0.6) (drill 0.3) (layers "F.Cu" "B.Cu") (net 2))
 (via (at 110.2 152) (size 0.6) (drill 0.3) (layers "F.Cu" "B.Cu") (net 2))
 (via (at 114.2 152) (size 0.6) (drill 0.3) (layers "F.Cu" "B.Cu") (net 2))
 (via (at 130.2 152) (size 0.6) (drill 0.3) (layers "F.Cu" "B.Cu") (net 2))
 (via (at 134.2 152) (size 0.6) (drill 0.3) (layers "F.Cu" "B.Cu") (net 2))
 (via (at 138.2 152) (size 0.6) (drill 0.3) (layers "F.Cu" "B.Cu") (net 2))
 (via (at 142.2 152) (size 0.6) (drill 0.3) (layers "F.Cu" "B.Cu") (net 2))
 (via (at 118.525 152.45) (size 0.6) (drill 0.3) (layers "F.Cu" "B.Cu") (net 2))
 (via (at 118.525 154.05) (size 0.6) (drill 0.3) (layers "F.Cu" "B.Cu") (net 2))
 (via (at 116.525 152.45) (size 0.6) (drill 0.3) (layers "F.Cu" "B.Cu") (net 2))
 (via (at 116.525 154.05) (size 0.6) (drill 0.3) (layers "F.Cu" "B.Cu") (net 2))
 (via (at 126.475 152.45) (size 0.6) (drill 0.3) (layers "F.Cu" "B.Cu") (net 2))
 (via (at 126.475 154.05) (size 0.6) (drill 0.3) (layers "F.Cu" "B.Cu") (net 2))
 (via (at 128.475 152.45) (size 0.6) (drill 0.3) (layers "F.Cu" "B.Cu") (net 2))
 (via (at 128.475 154.05) (size 0.6) (drill 0.3) (layers "F.Cu" "B.Cu") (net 2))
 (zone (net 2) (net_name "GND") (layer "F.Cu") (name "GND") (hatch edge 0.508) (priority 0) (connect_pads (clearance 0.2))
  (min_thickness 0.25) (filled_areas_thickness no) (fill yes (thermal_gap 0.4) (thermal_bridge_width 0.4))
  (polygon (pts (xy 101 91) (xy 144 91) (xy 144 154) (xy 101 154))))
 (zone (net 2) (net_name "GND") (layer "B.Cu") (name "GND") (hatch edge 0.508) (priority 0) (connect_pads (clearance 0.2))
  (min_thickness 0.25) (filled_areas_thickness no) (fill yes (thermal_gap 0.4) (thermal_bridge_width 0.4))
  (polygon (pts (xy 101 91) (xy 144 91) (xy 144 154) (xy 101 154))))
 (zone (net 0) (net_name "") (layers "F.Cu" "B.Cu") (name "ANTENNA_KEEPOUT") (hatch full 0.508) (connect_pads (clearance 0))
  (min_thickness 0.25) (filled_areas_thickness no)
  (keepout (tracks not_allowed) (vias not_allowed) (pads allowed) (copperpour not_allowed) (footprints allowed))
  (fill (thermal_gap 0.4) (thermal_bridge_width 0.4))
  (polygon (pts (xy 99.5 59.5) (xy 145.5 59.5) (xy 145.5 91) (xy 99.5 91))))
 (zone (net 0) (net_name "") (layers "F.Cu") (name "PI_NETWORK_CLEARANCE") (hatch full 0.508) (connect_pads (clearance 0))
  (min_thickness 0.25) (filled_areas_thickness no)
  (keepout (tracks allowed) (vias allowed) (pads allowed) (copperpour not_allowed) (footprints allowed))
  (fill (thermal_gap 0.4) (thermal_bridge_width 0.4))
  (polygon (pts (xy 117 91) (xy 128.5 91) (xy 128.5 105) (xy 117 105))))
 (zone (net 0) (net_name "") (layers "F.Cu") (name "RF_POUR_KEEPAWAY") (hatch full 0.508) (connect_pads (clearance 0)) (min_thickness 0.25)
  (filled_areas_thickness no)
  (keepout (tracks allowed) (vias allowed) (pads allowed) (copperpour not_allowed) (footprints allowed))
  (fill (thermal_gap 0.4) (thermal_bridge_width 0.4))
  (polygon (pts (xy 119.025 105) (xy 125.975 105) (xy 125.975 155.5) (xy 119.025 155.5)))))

